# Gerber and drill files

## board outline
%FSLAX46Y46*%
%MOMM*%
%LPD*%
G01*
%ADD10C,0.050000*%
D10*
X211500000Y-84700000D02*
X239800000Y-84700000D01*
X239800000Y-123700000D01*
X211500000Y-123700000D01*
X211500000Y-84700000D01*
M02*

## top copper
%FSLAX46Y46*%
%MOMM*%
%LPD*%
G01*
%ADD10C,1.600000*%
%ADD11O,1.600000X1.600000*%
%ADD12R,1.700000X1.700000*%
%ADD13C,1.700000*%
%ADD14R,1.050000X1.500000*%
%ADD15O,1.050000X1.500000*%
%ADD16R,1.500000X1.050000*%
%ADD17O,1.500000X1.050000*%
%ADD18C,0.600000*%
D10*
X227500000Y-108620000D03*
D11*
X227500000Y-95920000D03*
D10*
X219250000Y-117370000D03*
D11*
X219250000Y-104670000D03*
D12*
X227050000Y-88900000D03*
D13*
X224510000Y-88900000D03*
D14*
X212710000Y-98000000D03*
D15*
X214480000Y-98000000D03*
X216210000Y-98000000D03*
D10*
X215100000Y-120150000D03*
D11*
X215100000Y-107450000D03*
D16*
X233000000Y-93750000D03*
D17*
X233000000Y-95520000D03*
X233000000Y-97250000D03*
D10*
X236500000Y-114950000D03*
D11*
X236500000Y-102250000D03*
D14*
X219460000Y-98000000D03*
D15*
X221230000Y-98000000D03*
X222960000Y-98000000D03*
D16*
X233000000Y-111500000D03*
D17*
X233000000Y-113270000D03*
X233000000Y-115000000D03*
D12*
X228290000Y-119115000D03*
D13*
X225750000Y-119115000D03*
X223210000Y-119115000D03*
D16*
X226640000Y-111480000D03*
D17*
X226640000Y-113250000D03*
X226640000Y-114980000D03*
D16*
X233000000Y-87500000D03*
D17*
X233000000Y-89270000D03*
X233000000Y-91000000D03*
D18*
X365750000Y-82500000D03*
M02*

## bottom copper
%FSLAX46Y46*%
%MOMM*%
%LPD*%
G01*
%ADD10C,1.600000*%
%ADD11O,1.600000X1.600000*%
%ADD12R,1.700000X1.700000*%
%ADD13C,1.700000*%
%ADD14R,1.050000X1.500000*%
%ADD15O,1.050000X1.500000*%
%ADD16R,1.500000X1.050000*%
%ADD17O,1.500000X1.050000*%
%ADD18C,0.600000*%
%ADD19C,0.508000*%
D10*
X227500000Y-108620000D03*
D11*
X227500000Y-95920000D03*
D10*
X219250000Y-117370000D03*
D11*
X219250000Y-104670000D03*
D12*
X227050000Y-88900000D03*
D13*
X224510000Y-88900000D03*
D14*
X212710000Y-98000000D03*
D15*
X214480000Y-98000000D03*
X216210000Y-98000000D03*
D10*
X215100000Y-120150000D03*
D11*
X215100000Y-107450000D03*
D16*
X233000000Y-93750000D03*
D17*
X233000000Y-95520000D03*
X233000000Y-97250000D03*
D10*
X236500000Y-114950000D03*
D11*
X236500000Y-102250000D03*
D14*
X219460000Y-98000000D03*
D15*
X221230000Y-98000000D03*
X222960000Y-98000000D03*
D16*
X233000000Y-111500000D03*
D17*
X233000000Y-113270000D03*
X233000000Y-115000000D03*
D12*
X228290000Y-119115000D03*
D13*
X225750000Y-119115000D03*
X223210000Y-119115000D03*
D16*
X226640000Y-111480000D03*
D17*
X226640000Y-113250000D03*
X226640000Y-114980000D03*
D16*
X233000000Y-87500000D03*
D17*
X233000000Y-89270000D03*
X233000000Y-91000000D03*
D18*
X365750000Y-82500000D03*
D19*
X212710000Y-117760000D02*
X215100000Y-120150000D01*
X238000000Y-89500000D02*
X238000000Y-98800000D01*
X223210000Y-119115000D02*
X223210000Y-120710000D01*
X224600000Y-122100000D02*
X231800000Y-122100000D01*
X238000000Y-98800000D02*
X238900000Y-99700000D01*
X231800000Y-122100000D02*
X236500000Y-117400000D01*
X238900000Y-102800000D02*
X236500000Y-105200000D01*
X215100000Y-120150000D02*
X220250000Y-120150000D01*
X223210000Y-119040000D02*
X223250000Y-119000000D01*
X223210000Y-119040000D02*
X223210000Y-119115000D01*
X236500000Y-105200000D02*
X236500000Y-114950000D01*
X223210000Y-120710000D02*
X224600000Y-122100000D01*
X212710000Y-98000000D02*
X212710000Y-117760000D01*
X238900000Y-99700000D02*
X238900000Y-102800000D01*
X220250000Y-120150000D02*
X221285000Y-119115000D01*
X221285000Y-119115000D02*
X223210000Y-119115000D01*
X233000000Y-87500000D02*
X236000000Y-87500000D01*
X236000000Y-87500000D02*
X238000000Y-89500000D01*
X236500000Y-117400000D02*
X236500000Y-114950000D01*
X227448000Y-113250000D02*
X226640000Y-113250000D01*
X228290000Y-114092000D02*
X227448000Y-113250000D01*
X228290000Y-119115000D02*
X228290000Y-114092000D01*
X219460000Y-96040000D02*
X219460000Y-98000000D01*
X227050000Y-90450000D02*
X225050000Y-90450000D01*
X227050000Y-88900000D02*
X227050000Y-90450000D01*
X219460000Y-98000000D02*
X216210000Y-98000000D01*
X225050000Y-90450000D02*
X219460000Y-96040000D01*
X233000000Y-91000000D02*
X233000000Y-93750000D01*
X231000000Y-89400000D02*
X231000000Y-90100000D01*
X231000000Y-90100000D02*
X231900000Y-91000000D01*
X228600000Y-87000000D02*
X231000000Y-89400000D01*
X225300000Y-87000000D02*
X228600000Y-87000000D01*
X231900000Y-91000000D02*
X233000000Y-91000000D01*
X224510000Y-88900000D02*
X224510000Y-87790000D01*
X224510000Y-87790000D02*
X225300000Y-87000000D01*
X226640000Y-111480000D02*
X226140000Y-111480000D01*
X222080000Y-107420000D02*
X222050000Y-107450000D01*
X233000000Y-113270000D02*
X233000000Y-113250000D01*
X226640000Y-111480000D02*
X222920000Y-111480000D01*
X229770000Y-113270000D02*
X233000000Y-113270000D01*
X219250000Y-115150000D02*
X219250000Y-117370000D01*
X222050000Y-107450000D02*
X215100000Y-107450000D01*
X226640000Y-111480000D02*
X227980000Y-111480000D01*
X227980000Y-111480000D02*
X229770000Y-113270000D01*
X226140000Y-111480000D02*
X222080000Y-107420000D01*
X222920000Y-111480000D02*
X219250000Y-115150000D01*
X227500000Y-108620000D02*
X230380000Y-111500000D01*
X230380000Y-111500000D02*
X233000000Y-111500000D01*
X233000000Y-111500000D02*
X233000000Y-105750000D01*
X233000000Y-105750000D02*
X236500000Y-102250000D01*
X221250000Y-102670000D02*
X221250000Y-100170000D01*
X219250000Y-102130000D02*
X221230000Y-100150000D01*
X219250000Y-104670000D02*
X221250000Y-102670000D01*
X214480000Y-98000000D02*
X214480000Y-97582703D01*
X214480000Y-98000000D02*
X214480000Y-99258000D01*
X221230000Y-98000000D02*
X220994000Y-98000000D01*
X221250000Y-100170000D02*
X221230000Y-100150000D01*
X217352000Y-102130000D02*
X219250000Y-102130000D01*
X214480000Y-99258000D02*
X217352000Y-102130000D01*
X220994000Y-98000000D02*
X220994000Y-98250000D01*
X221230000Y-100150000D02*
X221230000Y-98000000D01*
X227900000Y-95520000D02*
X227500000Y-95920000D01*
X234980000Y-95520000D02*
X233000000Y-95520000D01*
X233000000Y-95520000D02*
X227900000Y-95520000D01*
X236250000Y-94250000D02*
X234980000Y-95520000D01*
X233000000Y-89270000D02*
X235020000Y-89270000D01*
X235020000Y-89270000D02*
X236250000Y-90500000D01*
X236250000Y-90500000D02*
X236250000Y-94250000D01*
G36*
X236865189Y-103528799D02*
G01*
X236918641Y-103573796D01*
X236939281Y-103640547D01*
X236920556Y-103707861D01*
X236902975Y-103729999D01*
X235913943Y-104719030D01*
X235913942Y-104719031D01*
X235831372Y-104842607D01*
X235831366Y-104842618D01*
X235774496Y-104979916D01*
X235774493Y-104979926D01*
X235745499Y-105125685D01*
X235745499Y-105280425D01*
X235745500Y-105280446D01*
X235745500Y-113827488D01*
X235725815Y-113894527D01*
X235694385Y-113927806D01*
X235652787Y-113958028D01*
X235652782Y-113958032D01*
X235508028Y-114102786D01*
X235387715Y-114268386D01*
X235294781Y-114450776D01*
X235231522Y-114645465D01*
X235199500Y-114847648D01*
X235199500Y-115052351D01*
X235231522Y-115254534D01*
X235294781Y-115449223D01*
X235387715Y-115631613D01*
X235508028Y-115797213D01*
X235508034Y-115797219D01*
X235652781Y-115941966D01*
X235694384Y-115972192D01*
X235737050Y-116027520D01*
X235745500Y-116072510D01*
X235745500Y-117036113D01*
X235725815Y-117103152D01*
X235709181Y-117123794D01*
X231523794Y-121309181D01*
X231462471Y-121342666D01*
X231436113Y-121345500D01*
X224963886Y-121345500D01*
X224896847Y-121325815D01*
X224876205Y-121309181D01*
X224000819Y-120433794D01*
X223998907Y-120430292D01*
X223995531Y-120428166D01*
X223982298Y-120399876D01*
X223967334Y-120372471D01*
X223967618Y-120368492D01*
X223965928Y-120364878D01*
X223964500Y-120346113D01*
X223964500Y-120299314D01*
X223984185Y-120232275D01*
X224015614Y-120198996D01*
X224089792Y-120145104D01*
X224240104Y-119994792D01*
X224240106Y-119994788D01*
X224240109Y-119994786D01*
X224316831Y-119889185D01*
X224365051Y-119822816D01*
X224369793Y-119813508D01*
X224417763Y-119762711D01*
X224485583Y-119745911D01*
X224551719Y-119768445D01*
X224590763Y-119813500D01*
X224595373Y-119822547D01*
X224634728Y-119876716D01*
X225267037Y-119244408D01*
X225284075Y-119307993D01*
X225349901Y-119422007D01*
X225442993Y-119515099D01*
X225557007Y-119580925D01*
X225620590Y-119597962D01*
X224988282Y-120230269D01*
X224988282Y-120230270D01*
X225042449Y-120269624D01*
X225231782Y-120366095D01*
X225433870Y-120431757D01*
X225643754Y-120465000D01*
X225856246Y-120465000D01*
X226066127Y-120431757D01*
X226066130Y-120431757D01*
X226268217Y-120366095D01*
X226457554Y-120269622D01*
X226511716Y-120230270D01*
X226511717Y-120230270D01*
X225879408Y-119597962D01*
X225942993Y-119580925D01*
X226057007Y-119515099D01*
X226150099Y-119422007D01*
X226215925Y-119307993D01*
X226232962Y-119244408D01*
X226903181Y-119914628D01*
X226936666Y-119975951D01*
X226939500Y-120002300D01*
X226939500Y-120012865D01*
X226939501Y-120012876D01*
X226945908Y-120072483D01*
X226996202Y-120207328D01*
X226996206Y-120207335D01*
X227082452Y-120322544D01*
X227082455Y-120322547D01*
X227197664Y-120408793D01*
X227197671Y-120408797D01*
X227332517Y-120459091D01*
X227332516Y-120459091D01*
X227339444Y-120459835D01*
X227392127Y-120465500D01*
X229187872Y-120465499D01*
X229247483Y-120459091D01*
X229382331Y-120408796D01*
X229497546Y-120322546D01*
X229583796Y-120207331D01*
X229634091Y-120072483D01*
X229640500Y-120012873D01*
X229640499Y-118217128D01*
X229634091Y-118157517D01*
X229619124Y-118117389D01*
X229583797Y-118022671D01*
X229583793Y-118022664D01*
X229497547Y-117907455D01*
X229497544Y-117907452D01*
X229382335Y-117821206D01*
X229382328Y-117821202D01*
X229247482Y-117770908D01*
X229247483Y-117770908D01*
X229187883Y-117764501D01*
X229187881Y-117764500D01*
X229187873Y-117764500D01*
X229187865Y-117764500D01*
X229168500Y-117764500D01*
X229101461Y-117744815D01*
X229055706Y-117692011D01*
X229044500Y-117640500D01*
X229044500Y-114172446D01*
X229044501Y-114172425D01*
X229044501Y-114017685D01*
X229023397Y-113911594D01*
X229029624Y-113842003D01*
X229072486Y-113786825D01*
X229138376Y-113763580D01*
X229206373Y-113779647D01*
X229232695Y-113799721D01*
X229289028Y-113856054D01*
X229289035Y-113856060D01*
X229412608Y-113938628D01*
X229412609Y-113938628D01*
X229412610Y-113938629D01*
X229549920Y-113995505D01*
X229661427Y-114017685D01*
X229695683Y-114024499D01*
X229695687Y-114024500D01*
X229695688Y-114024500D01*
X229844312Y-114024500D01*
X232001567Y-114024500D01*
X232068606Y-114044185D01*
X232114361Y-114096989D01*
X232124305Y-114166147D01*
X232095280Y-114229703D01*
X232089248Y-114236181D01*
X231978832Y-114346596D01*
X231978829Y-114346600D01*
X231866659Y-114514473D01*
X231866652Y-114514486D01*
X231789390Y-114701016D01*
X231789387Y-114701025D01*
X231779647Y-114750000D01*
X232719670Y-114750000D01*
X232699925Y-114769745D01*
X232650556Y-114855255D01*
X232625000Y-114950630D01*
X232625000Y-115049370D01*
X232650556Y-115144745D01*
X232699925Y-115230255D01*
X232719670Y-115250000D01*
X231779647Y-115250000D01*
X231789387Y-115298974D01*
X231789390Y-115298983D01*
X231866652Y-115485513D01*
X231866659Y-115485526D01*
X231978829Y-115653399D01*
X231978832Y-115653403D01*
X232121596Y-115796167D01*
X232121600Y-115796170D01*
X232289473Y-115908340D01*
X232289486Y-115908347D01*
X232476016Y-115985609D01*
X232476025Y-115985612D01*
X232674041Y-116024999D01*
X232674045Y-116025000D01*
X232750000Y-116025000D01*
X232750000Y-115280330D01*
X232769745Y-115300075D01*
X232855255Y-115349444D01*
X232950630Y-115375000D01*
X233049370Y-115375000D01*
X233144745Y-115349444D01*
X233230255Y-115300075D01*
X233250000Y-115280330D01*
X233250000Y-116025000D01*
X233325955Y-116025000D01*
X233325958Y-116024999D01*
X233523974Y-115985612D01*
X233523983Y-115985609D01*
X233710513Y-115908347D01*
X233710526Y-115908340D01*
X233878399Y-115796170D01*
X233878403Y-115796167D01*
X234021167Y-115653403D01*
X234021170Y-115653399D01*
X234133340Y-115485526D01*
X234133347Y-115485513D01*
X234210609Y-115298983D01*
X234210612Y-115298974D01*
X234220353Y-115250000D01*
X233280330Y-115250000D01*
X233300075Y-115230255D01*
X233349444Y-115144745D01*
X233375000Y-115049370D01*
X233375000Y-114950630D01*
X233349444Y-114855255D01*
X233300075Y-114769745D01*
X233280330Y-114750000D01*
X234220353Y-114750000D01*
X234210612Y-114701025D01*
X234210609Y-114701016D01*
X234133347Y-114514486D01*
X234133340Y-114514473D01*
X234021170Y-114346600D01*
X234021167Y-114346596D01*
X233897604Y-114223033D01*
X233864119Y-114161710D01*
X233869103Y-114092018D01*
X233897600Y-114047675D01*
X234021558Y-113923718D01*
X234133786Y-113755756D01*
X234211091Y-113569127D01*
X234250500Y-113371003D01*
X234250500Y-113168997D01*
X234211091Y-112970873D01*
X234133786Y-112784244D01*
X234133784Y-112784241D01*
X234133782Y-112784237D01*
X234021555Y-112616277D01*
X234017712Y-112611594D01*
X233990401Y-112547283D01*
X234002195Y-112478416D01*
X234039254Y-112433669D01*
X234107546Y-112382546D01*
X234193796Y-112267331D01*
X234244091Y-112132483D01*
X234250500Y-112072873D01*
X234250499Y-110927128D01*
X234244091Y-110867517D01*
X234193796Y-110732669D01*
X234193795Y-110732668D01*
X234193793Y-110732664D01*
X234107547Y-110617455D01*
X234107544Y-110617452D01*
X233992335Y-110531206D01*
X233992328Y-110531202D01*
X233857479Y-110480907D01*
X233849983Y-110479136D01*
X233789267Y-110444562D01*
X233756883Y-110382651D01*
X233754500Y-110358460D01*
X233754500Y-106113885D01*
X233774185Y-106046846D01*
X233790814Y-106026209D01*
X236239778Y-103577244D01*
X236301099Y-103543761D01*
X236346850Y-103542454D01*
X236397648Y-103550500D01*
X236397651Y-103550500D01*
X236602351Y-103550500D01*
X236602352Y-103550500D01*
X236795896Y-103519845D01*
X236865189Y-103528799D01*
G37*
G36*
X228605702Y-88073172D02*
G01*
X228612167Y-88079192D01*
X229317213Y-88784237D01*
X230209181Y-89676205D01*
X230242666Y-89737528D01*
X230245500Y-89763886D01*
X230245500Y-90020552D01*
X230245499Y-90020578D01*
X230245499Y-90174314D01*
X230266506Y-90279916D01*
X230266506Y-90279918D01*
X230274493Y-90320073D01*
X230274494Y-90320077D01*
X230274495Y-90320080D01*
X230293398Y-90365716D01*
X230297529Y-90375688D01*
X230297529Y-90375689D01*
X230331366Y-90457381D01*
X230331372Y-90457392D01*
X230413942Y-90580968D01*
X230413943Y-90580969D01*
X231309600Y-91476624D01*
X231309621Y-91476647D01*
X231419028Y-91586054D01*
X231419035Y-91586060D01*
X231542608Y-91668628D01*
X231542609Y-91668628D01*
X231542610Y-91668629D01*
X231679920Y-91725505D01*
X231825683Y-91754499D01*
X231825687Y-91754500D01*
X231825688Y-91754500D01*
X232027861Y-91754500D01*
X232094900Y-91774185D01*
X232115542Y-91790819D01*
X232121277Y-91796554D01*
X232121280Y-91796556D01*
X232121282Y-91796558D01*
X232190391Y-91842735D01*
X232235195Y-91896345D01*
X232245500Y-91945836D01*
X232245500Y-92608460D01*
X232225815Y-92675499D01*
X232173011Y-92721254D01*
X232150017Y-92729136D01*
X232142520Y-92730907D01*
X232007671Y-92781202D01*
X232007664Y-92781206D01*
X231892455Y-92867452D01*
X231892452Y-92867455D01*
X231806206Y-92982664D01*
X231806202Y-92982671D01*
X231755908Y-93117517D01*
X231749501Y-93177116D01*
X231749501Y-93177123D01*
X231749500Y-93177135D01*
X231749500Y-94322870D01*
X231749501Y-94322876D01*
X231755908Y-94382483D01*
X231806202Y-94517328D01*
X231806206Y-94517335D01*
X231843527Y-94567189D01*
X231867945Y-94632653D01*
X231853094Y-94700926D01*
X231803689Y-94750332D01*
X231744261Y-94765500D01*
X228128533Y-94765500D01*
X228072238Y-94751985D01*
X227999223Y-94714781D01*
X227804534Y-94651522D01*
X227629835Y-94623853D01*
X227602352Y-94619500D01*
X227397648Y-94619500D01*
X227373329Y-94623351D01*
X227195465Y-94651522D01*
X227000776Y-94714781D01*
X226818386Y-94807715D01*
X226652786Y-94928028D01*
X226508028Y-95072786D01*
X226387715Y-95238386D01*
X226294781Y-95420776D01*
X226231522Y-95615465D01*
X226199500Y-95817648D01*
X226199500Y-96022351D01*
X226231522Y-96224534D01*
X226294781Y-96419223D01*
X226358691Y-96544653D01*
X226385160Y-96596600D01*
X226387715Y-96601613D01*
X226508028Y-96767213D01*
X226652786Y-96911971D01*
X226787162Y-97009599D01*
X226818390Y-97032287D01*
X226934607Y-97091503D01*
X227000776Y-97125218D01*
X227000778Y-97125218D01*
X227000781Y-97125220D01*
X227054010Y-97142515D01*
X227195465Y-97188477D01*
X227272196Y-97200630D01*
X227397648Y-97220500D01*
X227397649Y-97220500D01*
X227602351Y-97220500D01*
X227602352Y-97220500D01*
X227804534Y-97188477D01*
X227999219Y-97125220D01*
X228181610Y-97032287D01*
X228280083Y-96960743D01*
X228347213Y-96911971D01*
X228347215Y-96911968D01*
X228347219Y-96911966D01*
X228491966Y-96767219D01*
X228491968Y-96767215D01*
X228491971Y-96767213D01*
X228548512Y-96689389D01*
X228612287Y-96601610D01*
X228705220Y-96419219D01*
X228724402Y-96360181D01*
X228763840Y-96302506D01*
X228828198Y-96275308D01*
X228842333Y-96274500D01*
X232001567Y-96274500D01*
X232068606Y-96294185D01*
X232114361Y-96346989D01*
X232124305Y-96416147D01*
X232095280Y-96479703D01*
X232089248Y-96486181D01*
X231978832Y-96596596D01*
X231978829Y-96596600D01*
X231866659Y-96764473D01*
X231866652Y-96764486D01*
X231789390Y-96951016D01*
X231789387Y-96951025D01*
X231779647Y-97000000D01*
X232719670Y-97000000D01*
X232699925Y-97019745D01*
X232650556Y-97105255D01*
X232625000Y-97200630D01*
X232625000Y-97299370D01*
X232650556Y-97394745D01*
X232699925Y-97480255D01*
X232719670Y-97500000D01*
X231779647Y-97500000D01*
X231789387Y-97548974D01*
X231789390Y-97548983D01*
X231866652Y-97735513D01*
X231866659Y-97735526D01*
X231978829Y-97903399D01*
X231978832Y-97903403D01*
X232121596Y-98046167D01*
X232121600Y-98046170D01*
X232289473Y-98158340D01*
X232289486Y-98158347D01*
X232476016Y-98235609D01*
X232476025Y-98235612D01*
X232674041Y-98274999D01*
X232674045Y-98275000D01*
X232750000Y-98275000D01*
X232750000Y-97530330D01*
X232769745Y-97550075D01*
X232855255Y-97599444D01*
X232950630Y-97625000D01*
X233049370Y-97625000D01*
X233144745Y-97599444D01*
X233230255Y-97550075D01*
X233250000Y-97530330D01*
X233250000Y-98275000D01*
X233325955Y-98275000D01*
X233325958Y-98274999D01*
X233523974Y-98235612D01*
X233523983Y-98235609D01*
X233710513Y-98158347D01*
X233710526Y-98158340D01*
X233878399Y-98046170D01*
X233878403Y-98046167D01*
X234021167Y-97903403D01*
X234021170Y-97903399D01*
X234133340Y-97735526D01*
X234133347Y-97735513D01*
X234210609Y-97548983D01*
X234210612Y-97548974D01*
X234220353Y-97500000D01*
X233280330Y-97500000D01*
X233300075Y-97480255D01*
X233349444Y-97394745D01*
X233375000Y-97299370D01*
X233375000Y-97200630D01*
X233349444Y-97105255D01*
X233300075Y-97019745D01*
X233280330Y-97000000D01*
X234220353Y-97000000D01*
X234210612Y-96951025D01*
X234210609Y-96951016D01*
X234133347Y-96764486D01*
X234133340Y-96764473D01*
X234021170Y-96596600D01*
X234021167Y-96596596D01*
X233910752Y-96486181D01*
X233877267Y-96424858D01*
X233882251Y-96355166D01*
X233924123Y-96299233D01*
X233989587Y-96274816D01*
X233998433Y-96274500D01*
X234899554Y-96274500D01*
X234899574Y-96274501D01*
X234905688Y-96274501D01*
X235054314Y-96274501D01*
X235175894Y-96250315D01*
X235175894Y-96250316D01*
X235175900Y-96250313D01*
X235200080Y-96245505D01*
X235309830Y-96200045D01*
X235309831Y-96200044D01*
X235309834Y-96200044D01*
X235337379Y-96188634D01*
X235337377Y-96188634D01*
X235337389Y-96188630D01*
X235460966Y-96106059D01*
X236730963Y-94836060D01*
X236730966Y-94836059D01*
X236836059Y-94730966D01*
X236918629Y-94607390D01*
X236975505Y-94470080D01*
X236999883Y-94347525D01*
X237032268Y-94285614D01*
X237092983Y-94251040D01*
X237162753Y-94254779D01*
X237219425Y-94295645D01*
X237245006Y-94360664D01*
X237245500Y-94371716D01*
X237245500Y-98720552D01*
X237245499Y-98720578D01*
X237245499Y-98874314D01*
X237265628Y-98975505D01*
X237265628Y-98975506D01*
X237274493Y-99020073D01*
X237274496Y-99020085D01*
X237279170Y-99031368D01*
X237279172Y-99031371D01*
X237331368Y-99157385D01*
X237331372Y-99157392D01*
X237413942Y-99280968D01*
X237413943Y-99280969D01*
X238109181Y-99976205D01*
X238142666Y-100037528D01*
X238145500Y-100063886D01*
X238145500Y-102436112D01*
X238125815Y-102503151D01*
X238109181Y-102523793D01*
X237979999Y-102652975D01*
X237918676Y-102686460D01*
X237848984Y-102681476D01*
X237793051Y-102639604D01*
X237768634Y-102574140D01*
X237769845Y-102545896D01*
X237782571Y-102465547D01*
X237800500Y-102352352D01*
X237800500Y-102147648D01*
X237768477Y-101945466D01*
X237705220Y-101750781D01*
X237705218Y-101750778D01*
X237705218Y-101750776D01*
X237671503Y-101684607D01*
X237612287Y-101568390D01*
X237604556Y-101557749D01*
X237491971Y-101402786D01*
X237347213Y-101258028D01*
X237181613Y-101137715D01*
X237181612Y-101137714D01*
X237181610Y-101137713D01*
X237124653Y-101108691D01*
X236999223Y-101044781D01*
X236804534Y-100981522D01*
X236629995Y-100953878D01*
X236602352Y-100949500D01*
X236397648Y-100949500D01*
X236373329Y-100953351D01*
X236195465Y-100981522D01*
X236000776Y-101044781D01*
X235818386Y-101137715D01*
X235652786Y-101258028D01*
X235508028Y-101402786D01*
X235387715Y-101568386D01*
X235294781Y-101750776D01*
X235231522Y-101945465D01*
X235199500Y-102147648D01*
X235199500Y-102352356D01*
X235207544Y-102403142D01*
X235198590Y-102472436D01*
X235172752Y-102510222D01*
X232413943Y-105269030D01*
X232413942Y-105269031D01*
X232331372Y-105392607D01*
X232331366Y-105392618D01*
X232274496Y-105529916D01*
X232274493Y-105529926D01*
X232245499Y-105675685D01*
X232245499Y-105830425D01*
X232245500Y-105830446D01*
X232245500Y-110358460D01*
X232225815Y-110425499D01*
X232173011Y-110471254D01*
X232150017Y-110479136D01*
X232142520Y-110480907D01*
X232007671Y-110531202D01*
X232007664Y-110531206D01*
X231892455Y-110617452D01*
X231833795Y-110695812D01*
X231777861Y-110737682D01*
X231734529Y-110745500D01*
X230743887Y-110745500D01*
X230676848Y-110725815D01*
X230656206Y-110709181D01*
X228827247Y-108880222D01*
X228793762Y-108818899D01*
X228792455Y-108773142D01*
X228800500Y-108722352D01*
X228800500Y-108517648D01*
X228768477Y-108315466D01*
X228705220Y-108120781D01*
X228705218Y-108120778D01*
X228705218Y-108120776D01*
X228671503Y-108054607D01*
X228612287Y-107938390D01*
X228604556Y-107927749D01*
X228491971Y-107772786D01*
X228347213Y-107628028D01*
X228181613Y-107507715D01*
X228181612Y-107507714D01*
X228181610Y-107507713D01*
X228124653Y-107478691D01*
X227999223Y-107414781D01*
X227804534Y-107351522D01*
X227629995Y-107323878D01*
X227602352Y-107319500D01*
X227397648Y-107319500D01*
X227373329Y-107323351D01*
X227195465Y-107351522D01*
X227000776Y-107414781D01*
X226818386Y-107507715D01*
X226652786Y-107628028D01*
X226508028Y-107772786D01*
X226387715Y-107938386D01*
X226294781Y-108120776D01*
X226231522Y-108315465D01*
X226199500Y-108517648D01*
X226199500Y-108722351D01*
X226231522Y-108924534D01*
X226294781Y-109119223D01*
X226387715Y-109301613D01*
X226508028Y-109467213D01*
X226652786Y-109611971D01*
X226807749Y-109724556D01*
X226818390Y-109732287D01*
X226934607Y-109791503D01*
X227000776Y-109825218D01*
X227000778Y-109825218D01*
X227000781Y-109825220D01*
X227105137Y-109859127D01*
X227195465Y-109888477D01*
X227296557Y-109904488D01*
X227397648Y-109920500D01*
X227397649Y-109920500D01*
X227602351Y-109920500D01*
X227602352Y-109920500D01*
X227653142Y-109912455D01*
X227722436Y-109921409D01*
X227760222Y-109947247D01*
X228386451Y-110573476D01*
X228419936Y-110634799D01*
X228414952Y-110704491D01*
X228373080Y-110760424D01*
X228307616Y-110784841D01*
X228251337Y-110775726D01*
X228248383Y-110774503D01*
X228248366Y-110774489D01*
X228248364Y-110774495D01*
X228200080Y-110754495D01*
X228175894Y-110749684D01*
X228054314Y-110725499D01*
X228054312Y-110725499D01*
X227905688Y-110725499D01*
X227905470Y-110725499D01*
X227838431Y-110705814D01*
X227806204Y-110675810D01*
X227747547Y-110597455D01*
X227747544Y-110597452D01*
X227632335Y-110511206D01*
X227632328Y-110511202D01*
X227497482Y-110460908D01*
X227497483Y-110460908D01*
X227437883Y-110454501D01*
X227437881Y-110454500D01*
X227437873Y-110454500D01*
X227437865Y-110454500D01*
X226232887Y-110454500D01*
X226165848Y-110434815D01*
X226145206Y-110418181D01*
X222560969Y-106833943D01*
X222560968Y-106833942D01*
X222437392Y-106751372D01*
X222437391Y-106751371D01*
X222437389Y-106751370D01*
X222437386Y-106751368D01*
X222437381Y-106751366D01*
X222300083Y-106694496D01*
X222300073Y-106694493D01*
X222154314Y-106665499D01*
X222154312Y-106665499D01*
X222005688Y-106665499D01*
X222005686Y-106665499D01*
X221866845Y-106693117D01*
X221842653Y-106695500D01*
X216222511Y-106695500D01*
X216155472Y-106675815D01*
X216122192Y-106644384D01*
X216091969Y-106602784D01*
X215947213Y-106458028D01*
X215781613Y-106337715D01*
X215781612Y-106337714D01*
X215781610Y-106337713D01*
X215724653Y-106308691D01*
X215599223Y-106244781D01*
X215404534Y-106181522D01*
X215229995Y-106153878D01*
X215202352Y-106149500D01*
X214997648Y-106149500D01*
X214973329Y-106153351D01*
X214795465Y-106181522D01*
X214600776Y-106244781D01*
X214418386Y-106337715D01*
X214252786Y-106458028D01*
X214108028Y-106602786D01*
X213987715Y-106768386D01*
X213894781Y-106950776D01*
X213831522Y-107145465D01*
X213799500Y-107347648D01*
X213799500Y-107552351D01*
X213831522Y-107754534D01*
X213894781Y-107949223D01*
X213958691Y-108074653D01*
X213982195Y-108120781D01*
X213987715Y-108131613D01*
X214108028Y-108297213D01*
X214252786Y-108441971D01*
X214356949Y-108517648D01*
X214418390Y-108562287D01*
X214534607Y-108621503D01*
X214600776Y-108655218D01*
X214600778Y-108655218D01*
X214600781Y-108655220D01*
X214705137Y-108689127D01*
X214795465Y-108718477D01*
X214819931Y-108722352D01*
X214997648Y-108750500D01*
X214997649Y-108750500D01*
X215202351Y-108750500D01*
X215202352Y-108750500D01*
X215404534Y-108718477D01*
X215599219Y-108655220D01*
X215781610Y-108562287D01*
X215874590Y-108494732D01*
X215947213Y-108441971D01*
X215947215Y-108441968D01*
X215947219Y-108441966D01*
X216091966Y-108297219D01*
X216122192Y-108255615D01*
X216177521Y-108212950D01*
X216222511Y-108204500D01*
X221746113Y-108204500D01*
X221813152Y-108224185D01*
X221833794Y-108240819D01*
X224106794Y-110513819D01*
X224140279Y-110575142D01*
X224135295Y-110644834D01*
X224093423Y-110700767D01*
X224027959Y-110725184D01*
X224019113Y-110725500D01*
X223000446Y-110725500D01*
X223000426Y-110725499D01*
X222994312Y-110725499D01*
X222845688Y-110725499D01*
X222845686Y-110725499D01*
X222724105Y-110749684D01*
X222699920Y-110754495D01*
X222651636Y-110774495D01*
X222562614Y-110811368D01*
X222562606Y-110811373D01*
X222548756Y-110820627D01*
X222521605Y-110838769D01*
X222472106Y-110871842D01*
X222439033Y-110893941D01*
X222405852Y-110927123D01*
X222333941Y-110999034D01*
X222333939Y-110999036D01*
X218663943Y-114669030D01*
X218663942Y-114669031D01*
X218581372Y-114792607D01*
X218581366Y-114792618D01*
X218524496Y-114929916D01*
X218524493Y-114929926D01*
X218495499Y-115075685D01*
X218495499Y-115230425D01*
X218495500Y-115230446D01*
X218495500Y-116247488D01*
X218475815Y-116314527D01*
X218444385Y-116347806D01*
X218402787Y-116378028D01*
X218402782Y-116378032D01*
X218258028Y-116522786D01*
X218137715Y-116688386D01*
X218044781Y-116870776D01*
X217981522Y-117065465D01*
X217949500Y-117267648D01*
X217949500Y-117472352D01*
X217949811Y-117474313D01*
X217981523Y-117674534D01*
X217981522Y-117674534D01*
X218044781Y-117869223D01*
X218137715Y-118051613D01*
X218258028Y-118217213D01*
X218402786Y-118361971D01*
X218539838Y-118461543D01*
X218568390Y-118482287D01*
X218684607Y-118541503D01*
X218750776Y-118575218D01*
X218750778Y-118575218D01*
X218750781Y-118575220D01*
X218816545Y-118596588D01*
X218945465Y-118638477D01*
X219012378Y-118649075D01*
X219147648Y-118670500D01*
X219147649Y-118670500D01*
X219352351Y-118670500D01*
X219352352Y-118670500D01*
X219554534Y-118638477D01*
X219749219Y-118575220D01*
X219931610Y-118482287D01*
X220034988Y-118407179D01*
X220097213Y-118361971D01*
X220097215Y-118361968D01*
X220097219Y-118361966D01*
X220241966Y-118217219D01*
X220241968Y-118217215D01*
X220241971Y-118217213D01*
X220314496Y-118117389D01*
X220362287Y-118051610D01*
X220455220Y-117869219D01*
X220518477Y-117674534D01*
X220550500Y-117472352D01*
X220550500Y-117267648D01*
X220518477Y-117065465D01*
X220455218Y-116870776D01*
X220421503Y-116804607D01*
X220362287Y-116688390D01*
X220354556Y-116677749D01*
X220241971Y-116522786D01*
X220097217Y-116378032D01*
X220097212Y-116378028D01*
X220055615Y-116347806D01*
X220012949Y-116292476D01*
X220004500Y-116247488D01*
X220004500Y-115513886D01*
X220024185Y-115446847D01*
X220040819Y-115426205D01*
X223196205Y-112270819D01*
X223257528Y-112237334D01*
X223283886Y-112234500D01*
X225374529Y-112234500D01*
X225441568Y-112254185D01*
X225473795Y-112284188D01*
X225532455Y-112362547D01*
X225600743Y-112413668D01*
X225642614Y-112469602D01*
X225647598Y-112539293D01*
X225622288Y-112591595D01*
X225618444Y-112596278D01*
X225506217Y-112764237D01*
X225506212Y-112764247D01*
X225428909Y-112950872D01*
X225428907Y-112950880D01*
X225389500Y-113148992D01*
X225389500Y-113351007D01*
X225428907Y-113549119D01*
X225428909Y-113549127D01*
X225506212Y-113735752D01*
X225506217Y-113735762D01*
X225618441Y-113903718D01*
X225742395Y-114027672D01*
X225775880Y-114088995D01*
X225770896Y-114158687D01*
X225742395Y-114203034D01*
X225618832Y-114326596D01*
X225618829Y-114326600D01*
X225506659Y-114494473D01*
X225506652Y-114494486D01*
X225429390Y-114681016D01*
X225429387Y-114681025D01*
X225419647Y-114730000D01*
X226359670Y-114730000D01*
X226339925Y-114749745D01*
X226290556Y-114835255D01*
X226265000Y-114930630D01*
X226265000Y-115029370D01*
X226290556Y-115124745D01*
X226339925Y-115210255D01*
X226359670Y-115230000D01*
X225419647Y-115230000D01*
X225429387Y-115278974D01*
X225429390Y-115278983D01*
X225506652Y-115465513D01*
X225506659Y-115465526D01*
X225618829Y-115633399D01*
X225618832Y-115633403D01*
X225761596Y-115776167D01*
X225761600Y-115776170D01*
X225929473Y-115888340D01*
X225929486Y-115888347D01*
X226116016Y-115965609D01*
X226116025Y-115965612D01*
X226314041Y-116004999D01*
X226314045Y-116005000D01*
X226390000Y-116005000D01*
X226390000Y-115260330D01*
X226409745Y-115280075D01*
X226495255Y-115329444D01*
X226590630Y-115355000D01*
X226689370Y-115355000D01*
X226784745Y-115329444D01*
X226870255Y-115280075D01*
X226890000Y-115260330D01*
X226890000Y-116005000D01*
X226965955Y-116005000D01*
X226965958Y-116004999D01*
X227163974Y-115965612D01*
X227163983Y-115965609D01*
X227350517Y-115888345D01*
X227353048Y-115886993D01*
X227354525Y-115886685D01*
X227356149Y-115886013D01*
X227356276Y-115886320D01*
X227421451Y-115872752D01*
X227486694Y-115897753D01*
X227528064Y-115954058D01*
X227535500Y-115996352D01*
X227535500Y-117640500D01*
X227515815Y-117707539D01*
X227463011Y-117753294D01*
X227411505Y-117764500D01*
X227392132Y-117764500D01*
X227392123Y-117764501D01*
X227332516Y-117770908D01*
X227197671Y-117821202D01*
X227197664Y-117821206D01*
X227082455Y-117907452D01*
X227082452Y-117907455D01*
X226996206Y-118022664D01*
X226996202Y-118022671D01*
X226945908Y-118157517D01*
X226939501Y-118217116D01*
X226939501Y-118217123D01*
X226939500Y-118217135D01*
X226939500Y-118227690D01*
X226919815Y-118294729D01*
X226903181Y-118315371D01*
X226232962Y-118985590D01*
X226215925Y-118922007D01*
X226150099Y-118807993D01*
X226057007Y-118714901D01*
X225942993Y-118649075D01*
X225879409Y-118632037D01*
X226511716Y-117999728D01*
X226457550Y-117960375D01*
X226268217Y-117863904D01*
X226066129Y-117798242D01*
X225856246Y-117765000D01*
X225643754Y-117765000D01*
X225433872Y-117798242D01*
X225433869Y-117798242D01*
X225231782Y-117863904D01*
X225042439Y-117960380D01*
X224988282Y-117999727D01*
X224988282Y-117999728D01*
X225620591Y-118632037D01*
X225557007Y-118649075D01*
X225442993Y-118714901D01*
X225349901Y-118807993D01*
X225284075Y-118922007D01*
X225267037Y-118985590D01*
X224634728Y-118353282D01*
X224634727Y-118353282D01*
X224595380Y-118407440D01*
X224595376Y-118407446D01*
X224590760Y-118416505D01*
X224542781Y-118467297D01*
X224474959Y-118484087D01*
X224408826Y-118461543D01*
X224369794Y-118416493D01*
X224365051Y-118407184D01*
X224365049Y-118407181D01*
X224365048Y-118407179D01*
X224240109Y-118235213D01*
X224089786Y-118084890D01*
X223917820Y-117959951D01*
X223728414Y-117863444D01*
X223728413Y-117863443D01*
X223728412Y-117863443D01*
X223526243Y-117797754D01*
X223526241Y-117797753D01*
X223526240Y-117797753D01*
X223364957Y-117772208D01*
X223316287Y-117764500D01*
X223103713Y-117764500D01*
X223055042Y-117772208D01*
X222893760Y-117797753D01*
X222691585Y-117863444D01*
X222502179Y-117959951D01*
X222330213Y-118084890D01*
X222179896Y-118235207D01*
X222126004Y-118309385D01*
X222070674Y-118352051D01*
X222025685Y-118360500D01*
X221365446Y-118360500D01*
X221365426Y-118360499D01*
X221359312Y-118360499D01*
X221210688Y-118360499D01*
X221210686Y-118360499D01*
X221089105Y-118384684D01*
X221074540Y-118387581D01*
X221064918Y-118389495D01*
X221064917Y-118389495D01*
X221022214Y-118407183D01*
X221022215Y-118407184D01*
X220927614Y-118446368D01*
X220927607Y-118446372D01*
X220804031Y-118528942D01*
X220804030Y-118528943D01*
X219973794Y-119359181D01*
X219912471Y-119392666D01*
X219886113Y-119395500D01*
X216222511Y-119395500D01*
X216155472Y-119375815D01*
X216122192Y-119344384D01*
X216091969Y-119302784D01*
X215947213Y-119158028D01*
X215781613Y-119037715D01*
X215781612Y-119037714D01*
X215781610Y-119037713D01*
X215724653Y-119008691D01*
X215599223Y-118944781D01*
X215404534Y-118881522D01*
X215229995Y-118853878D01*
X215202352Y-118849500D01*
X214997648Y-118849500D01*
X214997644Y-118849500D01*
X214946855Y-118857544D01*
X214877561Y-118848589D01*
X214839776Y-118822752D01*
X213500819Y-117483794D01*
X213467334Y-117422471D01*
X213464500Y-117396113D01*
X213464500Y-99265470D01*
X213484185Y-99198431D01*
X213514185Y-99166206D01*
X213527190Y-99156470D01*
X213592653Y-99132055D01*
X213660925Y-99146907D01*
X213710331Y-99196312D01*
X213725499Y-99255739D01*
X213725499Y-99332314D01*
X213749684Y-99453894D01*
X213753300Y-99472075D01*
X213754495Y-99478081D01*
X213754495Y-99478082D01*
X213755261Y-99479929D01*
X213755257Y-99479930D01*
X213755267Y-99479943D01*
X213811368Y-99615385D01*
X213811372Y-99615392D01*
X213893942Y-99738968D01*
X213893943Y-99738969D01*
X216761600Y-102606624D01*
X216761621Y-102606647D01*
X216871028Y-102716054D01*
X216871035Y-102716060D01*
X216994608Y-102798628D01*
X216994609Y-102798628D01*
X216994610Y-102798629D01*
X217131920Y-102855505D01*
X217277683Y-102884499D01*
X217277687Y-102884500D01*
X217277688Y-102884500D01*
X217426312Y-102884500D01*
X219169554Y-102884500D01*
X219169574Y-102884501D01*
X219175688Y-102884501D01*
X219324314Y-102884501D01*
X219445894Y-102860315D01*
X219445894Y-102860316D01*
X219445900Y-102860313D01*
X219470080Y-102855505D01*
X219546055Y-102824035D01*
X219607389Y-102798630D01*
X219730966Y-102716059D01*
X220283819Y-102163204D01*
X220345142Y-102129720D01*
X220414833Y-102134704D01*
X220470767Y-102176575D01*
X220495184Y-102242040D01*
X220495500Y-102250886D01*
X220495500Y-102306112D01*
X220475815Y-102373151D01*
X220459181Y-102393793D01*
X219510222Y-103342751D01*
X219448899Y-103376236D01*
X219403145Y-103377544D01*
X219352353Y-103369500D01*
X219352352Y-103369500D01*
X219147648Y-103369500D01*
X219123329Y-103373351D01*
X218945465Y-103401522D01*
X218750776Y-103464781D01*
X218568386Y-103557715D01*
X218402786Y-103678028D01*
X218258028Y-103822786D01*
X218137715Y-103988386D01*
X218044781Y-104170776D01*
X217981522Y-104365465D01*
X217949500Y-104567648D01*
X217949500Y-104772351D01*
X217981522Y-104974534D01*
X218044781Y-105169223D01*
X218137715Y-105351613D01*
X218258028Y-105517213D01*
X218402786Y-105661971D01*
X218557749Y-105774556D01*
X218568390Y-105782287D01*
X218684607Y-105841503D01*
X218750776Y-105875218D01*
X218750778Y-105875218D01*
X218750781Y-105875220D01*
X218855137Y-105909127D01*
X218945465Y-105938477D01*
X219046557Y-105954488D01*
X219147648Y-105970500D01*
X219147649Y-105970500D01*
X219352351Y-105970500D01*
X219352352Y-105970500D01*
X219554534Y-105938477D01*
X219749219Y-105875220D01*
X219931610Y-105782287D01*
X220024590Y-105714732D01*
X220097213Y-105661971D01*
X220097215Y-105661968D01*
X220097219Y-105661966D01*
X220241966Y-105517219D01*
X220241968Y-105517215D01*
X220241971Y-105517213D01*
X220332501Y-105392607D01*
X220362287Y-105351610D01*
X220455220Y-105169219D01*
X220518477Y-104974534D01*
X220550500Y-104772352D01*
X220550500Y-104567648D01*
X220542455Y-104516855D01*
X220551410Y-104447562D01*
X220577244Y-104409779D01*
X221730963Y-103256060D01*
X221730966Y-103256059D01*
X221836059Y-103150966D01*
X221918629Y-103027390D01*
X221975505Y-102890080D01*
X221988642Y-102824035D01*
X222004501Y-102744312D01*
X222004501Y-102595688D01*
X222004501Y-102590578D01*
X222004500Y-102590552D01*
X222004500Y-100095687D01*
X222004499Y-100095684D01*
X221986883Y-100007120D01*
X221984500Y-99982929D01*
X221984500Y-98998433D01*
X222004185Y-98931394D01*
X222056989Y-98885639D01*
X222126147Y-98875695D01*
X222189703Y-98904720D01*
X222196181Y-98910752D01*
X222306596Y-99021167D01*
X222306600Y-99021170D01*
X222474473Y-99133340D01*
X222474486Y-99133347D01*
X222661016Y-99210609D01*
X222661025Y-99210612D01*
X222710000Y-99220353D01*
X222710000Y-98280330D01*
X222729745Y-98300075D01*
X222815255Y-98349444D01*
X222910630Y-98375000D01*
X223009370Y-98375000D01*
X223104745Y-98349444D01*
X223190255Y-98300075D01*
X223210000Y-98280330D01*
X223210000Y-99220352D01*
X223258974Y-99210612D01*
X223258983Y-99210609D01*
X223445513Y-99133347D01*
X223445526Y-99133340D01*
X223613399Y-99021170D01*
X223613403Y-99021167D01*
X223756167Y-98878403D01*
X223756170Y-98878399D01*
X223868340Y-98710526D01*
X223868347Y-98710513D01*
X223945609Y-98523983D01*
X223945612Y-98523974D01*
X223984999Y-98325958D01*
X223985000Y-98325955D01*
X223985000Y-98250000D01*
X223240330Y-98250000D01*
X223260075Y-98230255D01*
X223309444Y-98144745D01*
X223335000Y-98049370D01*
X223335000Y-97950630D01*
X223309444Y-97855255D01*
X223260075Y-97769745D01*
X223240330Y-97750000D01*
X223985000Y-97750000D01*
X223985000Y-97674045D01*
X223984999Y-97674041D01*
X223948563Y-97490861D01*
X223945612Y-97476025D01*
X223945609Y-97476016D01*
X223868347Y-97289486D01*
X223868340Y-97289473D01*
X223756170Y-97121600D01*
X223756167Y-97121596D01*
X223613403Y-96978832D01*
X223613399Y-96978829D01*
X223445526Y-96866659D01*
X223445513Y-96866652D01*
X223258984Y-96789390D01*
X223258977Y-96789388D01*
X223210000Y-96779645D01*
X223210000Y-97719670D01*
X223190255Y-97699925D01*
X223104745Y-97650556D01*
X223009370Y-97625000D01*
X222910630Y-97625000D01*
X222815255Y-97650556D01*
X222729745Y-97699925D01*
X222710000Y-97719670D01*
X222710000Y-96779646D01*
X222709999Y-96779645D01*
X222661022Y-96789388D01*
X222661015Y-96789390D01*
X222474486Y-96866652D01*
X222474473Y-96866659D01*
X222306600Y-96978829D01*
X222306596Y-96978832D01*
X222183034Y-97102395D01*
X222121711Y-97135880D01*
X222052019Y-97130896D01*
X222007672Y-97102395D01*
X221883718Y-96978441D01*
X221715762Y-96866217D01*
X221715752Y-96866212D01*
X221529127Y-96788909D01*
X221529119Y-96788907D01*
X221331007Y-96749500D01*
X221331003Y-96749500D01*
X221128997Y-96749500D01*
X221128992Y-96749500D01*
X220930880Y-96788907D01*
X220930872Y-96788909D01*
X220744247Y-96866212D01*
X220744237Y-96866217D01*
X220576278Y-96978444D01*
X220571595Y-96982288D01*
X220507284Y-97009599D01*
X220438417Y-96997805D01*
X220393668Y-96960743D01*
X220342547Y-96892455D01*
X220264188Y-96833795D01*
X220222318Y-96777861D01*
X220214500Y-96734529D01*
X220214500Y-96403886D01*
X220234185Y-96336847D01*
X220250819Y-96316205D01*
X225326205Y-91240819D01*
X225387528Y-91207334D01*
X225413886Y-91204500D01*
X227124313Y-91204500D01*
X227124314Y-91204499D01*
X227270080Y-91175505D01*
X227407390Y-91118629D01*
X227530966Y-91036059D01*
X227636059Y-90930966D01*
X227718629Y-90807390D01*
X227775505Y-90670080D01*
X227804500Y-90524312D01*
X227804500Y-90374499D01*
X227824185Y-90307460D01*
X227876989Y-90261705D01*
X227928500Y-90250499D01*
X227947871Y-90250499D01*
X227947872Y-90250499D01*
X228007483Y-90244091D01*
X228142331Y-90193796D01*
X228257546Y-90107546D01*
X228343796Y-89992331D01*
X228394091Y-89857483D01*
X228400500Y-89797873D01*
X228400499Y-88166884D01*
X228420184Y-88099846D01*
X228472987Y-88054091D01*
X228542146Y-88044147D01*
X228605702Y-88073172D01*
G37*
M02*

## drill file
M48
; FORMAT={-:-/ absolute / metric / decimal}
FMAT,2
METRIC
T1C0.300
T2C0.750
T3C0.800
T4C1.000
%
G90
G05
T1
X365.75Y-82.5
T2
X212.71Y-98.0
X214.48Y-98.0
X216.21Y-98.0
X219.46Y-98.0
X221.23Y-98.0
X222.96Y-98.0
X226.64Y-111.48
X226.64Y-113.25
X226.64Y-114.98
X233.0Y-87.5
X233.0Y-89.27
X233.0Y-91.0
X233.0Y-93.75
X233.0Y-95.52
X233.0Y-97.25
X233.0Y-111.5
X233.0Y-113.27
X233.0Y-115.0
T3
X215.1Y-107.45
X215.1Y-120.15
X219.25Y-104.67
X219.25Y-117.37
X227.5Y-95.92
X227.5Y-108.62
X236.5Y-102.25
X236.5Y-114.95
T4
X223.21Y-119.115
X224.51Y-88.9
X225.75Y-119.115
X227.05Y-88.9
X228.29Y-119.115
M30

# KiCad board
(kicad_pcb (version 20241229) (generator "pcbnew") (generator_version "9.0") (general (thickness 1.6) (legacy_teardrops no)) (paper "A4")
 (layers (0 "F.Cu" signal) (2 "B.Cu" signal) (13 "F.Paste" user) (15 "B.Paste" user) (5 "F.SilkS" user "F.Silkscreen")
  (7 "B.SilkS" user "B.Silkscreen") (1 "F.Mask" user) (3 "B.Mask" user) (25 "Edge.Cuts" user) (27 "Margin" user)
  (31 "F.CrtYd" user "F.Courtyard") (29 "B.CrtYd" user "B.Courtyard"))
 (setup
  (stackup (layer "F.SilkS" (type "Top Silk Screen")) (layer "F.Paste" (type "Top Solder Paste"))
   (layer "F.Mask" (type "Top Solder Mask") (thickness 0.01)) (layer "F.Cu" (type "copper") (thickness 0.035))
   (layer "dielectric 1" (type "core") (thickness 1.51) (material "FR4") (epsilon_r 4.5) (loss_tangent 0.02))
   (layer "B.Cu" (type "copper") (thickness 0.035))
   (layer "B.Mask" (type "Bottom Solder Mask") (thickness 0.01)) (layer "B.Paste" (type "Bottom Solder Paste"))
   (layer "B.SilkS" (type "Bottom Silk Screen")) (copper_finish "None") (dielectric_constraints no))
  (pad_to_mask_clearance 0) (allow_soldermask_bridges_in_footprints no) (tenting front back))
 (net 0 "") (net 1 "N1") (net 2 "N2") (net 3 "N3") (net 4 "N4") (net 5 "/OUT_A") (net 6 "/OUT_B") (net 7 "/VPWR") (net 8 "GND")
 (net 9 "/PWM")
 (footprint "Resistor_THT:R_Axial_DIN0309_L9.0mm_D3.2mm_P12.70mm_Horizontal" (layer "F.Cu") (at 227.5 108.62 90)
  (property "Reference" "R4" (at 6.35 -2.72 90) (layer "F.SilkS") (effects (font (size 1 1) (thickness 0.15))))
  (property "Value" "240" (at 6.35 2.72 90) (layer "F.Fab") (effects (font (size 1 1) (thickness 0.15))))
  (pad "1" thru_hole circle (at 0 0 90) (size 1.6 1.6) (drill 0.8) (layers "*.Cu" "*.Mask") (remove_unused_layers no) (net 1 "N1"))
  (pad "2" thru_hole oval (at 12.7 0 90) (size 1.6 1.6) (drill 0.8) (layers "*.Cu" "*.Mask") (remove_unused_layers no) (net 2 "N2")))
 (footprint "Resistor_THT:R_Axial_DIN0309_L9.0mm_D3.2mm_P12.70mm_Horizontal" (layer "F.Cu") (at 219.25 117.37 90)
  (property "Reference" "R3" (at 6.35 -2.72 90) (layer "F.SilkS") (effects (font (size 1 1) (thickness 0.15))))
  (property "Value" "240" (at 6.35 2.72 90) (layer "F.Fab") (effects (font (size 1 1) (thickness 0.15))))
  (pad "1" thru_hole circle (at 0 0 90) (size 1.6 1.6) (drill 0.8) (layers "*.Cu" "*.Mask") (remove_unused_layers no) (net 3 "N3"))
  (pad "2" thru_hole oval (at 12.7 0 90) (size 1.6 1.6) (drill 0.8) (layers "*.Cu" "*.Mask") (remove_unused_layers no) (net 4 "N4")))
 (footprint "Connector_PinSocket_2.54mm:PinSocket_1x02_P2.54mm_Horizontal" (layer "F.Cu") (at 227.05 88.9 -90)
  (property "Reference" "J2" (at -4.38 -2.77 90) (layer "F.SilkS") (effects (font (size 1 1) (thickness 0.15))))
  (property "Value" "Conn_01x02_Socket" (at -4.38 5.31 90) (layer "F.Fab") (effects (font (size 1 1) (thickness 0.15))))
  (pad "1" thru_hole rect (at 0 0 270) (size 1.7 1.7) (drill 1) (layers "*.Cu" "*.Mask") (remove_unused_layers no) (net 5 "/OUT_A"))
  (pad "2" thru_hole circle (at 0 2.54 270) (size 1.7 1.7) (drill 1) (layers "*.Cu" "*.Mask") (remove_unused_layers no) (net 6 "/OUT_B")))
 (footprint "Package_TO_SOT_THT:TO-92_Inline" (layer "F.Cu") (at 213.21 98)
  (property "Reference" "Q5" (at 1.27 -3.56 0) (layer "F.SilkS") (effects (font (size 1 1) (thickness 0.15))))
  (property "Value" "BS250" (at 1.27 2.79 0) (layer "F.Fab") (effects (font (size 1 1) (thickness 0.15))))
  (pad "1" thru_hole rect (at -0.5 0) (size 1.05 1.5) (drill 0.75) (layers "*.Cu" "*.Mask") (remove_unused_layers no) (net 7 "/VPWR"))
  (pad "2" thru_hole oval (at 1.27 0) (size 1.05 1.5) (drill 0.75) (layers "*.Cu" "*.Mask") (remove_unused_layers no) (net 4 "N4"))
  (pad "3" thru_hole oval (at 3 0) (size 1.05 1.5) (drill 0.75) (layers "*.Cu" "*.Mask") (remove_unused_layers no) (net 5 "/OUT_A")))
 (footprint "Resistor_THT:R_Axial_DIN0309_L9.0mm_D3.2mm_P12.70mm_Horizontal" (layer "F.Cu") (at 215.1 120.15 90)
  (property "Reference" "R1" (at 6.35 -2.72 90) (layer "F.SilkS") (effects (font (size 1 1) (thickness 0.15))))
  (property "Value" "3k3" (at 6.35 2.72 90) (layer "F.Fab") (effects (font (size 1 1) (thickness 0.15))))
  (pad "1" thru_hole circle (at 0 0 90) (size 1.6 1.6) (drill 0.8) (layers "*.Cu" "*.Mask") (remove_unused_layers no) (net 7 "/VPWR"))
  (pad "2" thru_hole oval (at 12.7 0 90) (size 1.6 1.6) (drill 0.8) (layers "*.Cu" "*.Mask") (remove_unused_layers no) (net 3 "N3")))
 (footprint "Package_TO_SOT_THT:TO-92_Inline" (layer "F.Cu") (at 233 94.25 -90)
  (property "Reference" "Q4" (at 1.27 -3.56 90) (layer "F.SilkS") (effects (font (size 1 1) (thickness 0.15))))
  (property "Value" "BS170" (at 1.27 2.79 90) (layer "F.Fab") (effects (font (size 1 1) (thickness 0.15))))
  (pad "1" thru_hole rect (at -0.5 0 270) (size 1.05 1.5) (drill 0.75) (layers "*.Cu" "*.Mask") (remove_unused_layers no) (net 6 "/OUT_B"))
  (pad "2" thru_hole oval (at 1.27 0 270) (size 1.05 1.5) (drill 0.75) (layers "*.Cu" "*.Mask") (remove_unused_layers no) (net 2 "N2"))
  (pad "3" thru_hole oval (at 3 0 270) (size 1.05 1.5) (drill 0.75) (layers "*.Cu" "*.Mask") (remove_unused_layers no) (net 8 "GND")))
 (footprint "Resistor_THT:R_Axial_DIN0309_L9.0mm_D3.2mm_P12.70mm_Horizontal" (layer "F.Cu") (at 236.5 114.95 90)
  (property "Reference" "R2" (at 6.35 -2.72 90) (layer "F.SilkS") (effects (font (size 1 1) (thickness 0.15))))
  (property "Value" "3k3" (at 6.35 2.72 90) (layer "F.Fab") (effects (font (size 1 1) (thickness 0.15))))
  (pad "1" thru_hole circle (at 0 0 90) (size 1.6 1.6) (drill 0.8) (layers "*.Cu" "*.Mask") (remove_unused_layers no) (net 7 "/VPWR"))
  (pad "2" thru_hole oval (at 12.7 0 90) (size 1.6 1.6) (drill 0.8) (layers "*.Cu" "*.Mask") (remove_unused_layers no) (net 1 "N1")))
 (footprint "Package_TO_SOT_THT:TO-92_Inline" (layer "F.Cu") (at 219.96 98)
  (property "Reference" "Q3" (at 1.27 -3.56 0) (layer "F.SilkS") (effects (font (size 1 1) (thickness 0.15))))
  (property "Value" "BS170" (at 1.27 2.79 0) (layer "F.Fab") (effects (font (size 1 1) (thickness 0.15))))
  (pad "1" thru_hole rect (at -0.5 0) (size 1.05 1.5) (drill 0.75) (layers "*.Cu" "*.Mask") (remove_unused_layers no) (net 5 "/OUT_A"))
  (pad "2" thru_hole oval (at 1.27 0) (size 1.05 1.5) (drill 0.75) (layers "*.Cu" "*.Mask") (remove_unused_layers no) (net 4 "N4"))
  (pad "3" thru_hole oval (at 3 0) (size 1.05 1.5) (drill 0.75) (layers "*.Cu" "*.Mask") (remove_unused_layers no) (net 8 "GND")))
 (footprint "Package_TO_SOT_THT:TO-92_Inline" (layer "F.Cu") (at 233 112 -90)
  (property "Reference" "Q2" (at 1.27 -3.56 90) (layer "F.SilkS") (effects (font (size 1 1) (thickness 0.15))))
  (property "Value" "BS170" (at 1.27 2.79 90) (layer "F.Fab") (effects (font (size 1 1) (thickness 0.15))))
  (pad "1" thru_hole rect (at -0.5 0 270) (size 1.05 1.5) (drill 0.75) (layers "*.Cu" "*.Mask") (remove_unused_layers no) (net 1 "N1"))
  (pad "2" thru_hole oval (at 1.27 0 270) (size 1.05 1.5) (drill 0.75) (layers "*.Cu" "*.Mask") (remove_unused_layers no) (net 3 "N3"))
  (pad "3" thru_hole oval (at 3 0 270) (size 1.05 1.5) (drill 0.75) (layers "*.Cu" "*.Mask") (remove_unused_layers no) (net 8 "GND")))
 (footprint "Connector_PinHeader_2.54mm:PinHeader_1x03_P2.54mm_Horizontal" (layer "F.Cu") (at 228.29 119.115 -90)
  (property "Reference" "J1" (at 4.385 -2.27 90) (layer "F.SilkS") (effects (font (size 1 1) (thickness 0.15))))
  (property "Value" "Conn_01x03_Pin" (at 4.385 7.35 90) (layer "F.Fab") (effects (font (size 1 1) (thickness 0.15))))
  (pad "1" thru_hole rect (at 0 0 270) (size 1.7 1.7) (drill 1) (layers "*.Cu" "*.Mask") (remove_unused_layers no) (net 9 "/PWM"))
  (pad "2" thru_hole circle (at 0 2.54 270) (size 1.7 1.7) (drill 1) (layers "*.Cu" "*.Mask") (remove_unused_layers no) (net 8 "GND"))
  (pad "3" thru_hole circle (at 0 5.08 270) (size 1.7 1.7) (drill 1) (layers "*.Cu" "*.Mask") (remove_unused_layers no) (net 7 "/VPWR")))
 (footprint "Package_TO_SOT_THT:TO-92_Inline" (layer "F.Cu") (at 226.64 111.98 -90)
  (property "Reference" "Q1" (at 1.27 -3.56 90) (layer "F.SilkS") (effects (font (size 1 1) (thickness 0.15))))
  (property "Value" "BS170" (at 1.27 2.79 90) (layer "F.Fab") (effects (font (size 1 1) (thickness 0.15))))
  (pad "1" thru_hole rect (at -0.5 0 270) (size 1.05 1.5) (drill 0.75) (layers "*.Cu" "*.Mask") (remove_unused_layers no) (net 3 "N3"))
  (pad "2" thru_hole oval (at 1.27 0 270) (size 1.05 1.5) (drill 0.75) (layers "*.Cu" "*.Mask") (remove_unused_layers no) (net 9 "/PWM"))
  (pad "3" thru_hole oval (at 3 0 270) (size 1.05 1.5) (drill 0.75) (layers "*.Cu" "*.Mask") (remove_unused_layers no) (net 8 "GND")))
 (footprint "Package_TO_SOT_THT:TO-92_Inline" (layer "F.Cu") (at 233 88 -90)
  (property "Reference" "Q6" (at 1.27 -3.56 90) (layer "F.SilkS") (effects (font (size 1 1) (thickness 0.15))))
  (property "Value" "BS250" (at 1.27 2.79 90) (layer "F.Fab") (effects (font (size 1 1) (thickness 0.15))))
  (pad "1" thru_hole rect (at -0.5 0 270) (size 1.05 1.5) (drill 0.75) (layers "*.Cu" "*.Mask") (remove_unused_layers no) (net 7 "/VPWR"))
  (pad "2" thru_hole oval (at 1.27 0 270) (size 1.05 1.5) (drill 0.75) (layers "*.Cu" "*.Mask") (remove_unused_layers no) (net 2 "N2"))
  (pad "3" thru_hole oval (at 3 0 270) (size 1.05 1.5) (drill 0.75) (layers "*.Cu" "*.Mask") (remove_unused_layers no) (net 6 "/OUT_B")))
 (gr_rect (start 211.5 84.7) (end 239.8 123.7) (stroke (width 0.05) (type default)) (fill no) (layer "Edge.Cuts"))
 (via (at 365.75 82.5) (size 0.6) (drill 0.3) (layers "F.Cu" "B.Cu") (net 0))
 (segment (start 212.71 117.76) (end 215.1 120.15) (width 0.508) (layer "B.Cu") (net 7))
 (segment (start 238 89.5) (end 238 98.8) (width 0.508) (layer "B.Cu") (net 7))
 (segment (start 223.21 119.115) (end 223.21 120.71) (width 0.508) (layer "B.Cu") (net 7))
 (segment (start 224.6 122.1) (end 231.8 122.1) (width 0.508) (layer "B.Cu") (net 7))
 (segment (start 238 98.8) (end 238.9 99.7) (width 0.508) (layer "B.Cu") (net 7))
 (segment (start 231.8 122.1) (end 236.5 117.4) (width 0.508) (layer "B.Cu") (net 7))
 (segment (start 238.9 102.8) (end 236.5 105.2) (width 0.508) (layer "B.Cu") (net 7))
 (segment (start 215.1 120.15) (end 220.25 120.15) (width 0.508) (layer "B.Cu") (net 7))
 (segment (start 223.21 119.04) (end 223.25 119) (width 0.508) (layer "B.Cu") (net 7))
 (segment (start 223.21 119.04) (end 223.21 119.115) (width 0.508) (layer "B.Cu") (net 7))
 (segment (start 236.5 105.2) (end 236.5 114.95) (width 0.508) (layer "B.Cu") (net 7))
 (segment (start 223.21 120.71) (end 224.6 122.1) (width 0.508) (layer "B.Cu") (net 7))
 (segment (start 212.71 98) (end 212.71 117.76) (width 0.508) (layer "B.Cu") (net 7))
 (segment (start 238.9 99.7) (end 238.9 102.8) (width 0.508) (layer "B.Cu") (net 7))
 (segment (start 220.25 120.15) (end 221.285 119.115) (width 0.508) (layer "B.Cu") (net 7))
 (segment (start 221.285 119.115) (end 223.21 119.115) (width 0.508) (layer "B.Cu") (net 7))
 (segment (start 233 87.5) (end 236 87.5) (width 0.508) (layer "B.Cu") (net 7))
 (segment (start 236 87.5) (end 238 89.5) (width 0.508) (layer "B.Cu") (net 7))
 (segment (start 236.5 117.4) (end 236.5 114.95) (width 0.508) (layer "B.Cu") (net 7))
 (segment (start 227.448 113.25) (end 226.64 113.25) (width 0.508) (layer "B.Cu") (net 9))
 (segment (start 228.29 114.092) (end 227.448 113.25) (width 0.508) (layer "B.Cu") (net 9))
 (segment (start 228.29 119.115) (end 228.29 114.092) (width 0.508) (layer "B.Cu") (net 9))
 (segment (start 219.46 96.04) (end 219.46 98) (width 0.508) (layer "B.Cu") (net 5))
 (segment (start 227.05 90.45) (end 225.05 90.45) (width 0.508) (layer "B.Cu") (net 5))
 (segment (start 227.05 88.9) (end 227.05 90.45) (width 0.508) (layer "B.Cu") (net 5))
 (segment (start 219.46 98) (end 216.21 98) (width 0.508) (layer "B.Cu") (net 5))
 (segment (start 225.05 90.45) (end 219.46 96.04) (width 0.508) (layer "B.Cu") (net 5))
 (segment (start 233 91) (end 233 93.75) (width 0.508) (layer "B.Cu") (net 6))
 (segment (start 231 89.4) (end 231 90.1) (width 0.508) (layer "B.Cu") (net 6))
 (segment (start 231 90.1) (end 231.9 91) (width 0.508) (layer "B.Cu") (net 6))
 (segment (start 228.6 87) (end 231 89.4) (width 0.508) (layer "B.Cu") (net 6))
 (segment (start 225.3 87) (end 228.6 87) (width 0.508) (layer "B.Cu") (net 6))
 (segment (start 231.9 91) (end 233 91) (width 0.508) (layer "B.Cu") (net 6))
 (segment (start 224.51 88.9) (end 224.51 87.79) (width 0.508) (layer "B.Cu") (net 6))
 (segment (start 224.51 87.79) (end 225.3 87) (width 0.508) (layer "B.Cu") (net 6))
 (segment (start 226.64 111.48) (end 226.14 111.48) (width 0.508) (layer "B.Cu") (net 3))
 (segment (start 222.08 107.42) (end 222.05 107.45) (width 0.508) (layer "B.Cu") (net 3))
 (segment (start 233 113.27) (end 233 113.25) (width 0.508) (layer "B.Cu") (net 3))
 (segment (start 226.64 111.48) (end 222.92 111.48) (width 0.508) (layer "B.Cu") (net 3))
 (segment (start 229.77 113.27) (end 233 113.27) (width 0.508) (layer "B.Cu") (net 3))
 (segment (start 219.25 115.15) (end 219.25 117.37) (width 0.508) (layer "B.Cu") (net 3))
 (segment (start 222.05 107.45) (end 215.1 107.45) (width 0.508) (layer "B.Cu") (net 3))
 (segment (start 226.64 111.48) (end 227.98 111.48) (width 0.508) (layer "B.Cu") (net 3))
 (segment (start 227.98 111.48) (end 229.77 113.27) (width 0.508) (layer "B.Cu") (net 3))
 (segment (start 226.14 111.48) (end 222.08 107.42) (width 0.508) (layer "B.Cu") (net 3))
 (segment (start 222.92 111.48) (end 219.25 115.15) (width 0.508) (layer "B.Cu") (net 3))
 (segment (start 227.5 108.62) (end 230.38 111.5) (width 0.508) (layer "B.Cu") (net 1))
 (segment (start 230.38 111.5) (end 233 111.5) (width 0.508) (layer "B.Cu") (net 1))
 (segment (start 233 111.5) (end 233 105.75) (width 0.508) (layer "B.Cu") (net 1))
 (segment (start 233 105.75) (end 236.5 102.25) (width 0.508) (layer "B.Cu") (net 1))
 (segment (start 221.25 102.67) (end 221.25 100.17) (width 0.508) (layer "B.Cu") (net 4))
 (segment (start 219.25 102.13) (end 221.23 100.15) (width 0.508) (layer "B.Cu") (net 4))
 (segment (start 219.25 104.67) (end 221.25 102.67) (width 0.508) (layer "B.Cu") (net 4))
 (segment (start 214.48 98) (end 214.48 97.582703) (width 0.508) (layer "B.Cu") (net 4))
 (segment (start 214.48 98) (end 214.48 99.258) (width 0.508) (layer "B.Cu") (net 4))
 (segment (start 221.23 98) (end 220.994 98) (width 0.508) (layer "B.Cu") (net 4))
 (segment (start 221.25 100.17) (end 221.23 100.15) (width 0.508) (layer "B.Cu") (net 4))
 (segment (start 217.352 102.13) (end 219.25 102.13) (width 0.508) (layer "B.Cu") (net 4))
 (segment (start 214.48 99.258) (end 217.352 102.13) (width 0.508) (layer "B.Cu") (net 4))
 (segment (start 220.994 98) (end 220.994 98.25) (width 0.508) (layer "B.Cu") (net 4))
 (segment (start 221.23 100.15) (end 221.23 98) (width 0.508) (layer "B.Cu") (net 4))
 (segment (start 227.9 95.52) (end 227.5 95.92) (width 0.508) (layer "B.Cu") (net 2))
 (segment (start 234.98 95.52) (end 233 95.52) (width 0.508) (layer "B.Cu") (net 2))
 (segment (start 233 95.52) (end 227.9 95.52) (width 0.508) (layer "B.Cu") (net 2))
 (segment (start 236.25 94.25) (end 234.98 95.52) (width 0.508) (layer "B.Cu") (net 2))
 (segment (start 233 89.27) (end 235.02 89.27) (width 0.508) (layer "B.Cu") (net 2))
 (segment (start 235.02 89.27) (end 236.25 90.5) (width 0.508) (layer "B.Cu") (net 2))
 (segment (start 236.25 90.5) (end 236.25 94.25) (width 0.508) (layer "B.Cu") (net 2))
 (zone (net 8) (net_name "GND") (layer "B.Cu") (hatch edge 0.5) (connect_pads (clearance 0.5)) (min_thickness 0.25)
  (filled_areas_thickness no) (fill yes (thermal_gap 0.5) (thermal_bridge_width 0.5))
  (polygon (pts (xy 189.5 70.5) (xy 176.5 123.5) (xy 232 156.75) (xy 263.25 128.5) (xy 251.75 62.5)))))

